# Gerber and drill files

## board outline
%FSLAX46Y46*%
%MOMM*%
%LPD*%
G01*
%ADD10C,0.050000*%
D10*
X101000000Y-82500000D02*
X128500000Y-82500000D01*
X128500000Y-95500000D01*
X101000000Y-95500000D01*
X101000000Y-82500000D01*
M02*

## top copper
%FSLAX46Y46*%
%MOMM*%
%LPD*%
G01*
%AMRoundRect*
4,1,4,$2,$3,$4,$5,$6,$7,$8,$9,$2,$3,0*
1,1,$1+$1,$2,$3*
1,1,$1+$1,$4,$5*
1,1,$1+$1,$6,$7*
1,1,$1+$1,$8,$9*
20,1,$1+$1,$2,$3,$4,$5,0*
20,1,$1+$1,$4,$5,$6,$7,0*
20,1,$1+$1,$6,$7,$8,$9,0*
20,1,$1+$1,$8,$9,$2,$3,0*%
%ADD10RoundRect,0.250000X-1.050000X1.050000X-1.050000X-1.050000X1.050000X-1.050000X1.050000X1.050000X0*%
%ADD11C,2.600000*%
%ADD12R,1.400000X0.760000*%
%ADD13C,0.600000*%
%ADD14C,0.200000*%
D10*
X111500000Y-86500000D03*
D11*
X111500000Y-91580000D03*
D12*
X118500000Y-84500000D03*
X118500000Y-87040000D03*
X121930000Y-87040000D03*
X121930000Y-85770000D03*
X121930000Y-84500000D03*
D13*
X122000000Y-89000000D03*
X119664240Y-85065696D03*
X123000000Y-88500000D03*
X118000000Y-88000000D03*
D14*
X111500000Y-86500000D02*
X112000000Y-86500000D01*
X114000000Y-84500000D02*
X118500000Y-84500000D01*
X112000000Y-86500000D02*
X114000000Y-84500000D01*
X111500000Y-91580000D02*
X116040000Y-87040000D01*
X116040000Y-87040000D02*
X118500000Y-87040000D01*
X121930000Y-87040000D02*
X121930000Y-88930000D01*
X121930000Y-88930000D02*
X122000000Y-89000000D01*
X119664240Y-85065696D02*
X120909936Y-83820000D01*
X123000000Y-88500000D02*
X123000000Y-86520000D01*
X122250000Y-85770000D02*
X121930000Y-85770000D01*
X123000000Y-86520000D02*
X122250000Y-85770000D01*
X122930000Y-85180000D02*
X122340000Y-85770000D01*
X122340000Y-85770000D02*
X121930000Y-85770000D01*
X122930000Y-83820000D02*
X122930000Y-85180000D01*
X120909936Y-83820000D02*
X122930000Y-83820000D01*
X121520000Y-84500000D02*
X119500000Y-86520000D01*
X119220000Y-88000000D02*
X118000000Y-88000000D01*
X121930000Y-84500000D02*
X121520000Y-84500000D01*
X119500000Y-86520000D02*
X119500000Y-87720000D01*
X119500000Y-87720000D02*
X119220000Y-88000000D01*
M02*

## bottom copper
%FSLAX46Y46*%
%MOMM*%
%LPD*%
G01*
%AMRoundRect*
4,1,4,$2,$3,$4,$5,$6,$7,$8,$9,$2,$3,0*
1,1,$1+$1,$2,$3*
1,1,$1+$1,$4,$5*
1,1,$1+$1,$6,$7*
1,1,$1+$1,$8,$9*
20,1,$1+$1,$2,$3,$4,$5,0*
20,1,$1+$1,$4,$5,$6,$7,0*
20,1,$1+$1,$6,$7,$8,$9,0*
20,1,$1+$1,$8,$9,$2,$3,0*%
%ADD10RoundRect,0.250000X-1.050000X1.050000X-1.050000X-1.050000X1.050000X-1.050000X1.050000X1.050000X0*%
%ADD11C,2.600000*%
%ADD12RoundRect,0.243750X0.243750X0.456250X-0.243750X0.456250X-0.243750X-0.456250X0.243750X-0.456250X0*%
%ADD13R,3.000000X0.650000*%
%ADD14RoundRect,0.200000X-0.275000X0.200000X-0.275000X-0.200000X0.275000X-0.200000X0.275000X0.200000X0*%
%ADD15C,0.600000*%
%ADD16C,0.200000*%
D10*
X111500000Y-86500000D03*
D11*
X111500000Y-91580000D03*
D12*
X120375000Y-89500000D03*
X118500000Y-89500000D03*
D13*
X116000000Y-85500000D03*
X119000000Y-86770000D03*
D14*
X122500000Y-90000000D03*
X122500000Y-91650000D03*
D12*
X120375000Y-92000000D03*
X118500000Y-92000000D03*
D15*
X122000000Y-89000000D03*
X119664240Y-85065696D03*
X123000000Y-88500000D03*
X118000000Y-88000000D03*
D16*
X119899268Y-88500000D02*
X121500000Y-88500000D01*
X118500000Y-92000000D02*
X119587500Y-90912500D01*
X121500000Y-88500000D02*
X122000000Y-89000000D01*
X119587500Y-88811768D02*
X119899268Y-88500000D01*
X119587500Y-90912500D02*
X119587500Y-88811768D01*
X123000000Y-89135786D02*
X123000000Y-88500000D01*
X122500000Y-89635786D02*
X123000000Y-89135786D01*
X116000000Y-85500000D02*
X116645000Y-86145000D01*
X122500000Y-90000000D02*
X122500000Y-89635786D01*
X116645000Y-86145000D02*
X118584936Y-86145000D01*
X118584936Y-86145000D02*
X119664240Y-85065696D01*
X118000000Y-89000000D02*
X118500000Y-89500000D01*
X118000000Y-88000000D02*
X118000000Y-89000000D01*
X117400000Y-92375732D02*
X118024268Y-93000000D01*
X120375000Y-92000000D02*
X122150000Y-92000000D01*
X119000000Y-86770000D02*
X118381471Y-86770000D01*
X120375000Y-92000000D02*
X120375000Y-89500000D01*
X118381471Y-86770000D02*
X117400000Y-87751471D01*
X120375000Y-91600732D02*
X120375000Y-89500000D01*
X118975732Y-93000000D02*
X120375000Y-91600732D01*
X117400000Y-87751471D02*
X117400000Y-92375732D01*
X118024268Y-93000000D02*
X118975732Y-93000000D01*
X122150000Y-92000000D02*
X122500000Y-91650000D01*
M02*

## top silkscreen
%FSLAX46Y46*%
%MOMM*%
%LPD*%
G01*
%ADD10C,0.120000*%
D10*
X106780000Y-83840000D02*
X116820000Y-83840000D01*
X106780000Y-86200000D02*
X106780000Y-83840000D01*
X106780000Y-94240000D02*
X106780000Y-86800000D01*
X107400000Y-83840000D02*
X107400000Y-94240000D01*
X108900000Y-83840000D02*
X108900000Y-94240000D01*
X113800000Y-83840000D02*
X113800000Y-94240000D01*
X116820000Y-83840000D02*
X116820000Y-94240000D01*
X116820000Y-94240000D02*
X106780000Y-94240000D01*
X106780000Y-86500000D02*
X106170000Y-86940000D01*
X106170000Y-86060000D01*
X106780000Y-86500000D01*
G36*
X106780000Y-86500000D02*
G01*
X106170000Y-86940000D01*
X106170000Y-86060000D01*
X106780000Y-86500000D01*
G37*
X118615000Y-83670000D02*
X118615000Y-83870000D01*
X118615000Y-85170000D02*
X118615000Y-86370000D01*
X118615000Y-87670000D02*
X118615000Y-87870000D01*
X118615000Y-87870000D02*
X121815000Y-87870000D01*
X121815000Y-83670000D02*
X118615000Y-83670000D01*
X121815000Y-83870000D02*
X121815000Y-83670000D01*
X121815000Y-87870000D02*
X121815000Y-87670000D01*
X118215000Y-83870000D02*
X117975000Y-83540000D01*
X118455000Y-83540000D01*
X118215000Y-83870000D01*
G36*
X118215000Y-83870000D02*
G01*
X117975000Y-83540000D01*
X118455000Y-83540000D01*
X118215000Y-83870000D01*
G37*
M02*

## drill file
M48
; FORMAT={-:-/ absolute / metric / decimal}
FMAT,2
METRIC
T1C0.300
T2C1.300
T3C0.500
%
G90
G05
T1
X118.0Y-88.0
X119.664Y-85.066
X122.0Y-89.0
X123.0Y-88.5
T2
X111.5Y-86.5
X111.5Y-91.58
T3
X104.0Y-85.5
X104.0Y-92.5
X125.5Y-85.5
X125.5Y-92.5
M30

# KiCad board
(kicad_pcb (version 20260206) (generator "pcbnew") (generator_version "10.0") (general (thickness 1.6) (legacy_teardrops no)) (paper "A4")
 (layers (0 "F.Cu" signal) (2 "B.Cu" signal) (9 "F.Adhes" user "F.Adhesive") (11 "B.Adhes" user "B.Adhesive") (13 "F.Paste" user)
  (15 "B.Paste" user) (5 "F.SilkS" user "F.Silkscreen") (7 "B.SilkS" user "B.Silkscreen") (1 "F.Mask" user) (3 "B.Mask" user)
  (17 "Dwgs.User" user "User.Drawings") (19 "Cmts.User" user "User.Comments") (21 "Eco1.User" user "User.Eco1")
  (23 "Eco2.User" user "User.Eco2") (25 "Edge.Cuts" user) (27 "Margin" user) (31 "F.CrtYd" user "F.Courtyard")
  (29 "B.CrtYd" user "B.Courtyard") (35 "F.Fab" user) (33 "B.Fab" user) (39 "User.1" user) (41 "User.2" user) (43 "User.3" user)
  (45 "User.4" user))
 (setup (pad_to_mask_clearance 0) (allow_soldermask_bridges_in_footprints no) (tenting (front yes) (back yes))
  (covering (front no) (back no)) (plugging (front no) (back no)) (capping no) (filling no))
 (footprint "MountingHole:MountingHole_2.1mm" (layer "F.Cu") (at 104 92.5)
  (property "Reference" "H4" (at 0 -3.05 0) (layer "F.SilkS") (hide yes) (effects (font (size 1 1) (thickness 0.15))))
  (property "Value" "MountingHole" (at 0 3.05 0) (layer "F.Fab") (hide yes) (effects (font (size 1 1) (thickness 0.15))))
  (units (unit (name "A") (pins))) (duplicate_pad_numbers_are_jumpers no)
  (pad "" np_thru_hole circle (at 0 0) (size 0.5 0.5) (drill 0.5) (layers "*.Cu" "*.Mask")))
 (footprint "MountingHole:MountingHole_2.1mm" (layer "F.Cu") (at 125.5 85.5)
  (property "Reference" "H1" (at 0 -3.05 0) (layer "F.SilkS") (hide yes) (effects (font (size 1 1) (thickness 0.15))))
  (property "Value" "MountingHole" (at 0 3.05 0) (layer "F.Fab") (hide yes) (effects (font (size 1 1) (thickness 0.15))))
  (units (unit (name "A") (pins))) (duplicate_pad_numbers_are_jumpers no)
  (pad "" np_thru_hole circle (at 0 0) (size 0.5 0.5) (drill 0.5) (layers "*.Cu" "*.Mask")))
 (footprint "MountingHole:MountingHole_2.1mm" (layer "F.Cu") (at 104 85.5)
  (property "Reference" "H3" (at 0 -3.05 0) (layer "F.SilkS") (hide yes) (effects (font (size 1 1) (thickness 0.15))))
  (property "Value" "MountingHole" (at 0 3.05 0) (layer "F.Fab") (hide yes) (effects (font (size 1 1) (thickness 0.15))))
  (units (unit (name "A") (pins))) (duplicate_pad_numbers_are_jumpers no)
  (pad "" np_thru_hole circle (at 0 0) (size 0.5 0.5) (drill 0.5) (layers "*.Cu" "*.Mask")))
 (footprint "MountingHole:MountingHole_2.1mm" (layer "F.Cu") (at 125.5 92.5)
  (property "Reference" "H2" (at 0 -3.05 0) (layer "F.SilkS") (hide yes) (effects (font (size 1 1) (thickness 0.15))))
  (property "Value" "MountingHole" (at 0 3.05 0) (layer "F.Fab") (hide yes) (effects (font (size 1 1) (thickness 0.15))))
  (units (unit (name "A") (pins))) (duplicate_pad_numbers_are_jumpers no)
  (pad "" np_thru_hole circle (at 0 0) (size 0.5 0.5) (drill 0.5) (layers "*.Cu" "*.Mask")))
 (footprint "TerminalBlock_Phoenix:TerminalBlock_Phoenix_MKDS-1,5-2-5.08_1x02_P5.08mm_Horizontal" (layer "F.Cu") (at 111.5 86.5 -90)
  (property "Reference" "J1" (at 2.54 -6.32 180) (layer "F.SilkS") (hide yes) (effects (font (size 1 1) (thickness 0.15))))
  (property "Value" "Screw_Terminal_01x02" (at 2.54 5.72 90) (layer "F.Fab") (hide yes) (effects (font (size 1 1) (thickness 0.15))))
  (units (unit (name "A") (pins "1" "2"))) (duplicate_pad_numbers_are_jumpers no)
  (fp_line (start -2.66 4.72) (end -2.66 -5.32) (stroke (width 0.12) (type solid)) (layer "F.SilkS"))
  (fp_line (start -0.3 4.72) (end -2.66 4.72) (stroke (width 0.12) (type solid)) (layer "F.SilkS"))
  (fp_line (start 7.74 4.72) (end 0.3 4.72) (stroke (width 0.12) (type solid)) (layer "F.SilkS"))
  (fp_line (start -2.66 4.1) (end 7.74 4.1) (stroke (width 0.12) (type solid)) (layer "F.SilkS"))
  (fp_line (start -2.66 2.6) (end 7.74 2.6) (stroke (width 0.12) (type solid)) (layer "F.SilkS"))
  (fp_line (start -2.66 -2.3) (end 7.74 -2.3) (stroke (width 0.12) (type solid)) (layer "F.SilkS"))
  (fp_line (start -2.66 -5.32) (end 7.74 -5.32) (stroke (width 0.12) (type solid)) (layer "F.SilkS"))
  (fp_line (start 7.74 -5.32) (end 7.74 4.72) (stroke (width 0.12) (type solid)) (layer "F.SilkS"))
  (fp_poly (pts (xy 0 4.72) (xy 0.44 5.33) (xy -0.44 5.33)) (stroke (width 0.12) (type solid)) (fill yes) (layer "F.SilkS"))
  (pad "1" thru_hole roundrect (at 0 0 270) (size 2.6 2.6) (drill 1.3) (layers "*.Cu" "*.Mask") (remove_unused_layers no)
   (roundrect_rratio 0.096154) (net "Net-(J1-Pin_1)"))
  (pad "2" thru_hole circle (at 5.08 0 270) (size 2.6 2.6) (drill 1.3) (layers "*.Cu" "*.Mask") (remove_unused_layers no)
   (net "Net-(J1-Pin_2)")))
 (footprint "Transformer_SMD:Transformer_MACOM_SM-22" (layer "F.Cu") (at 120.215 85.77)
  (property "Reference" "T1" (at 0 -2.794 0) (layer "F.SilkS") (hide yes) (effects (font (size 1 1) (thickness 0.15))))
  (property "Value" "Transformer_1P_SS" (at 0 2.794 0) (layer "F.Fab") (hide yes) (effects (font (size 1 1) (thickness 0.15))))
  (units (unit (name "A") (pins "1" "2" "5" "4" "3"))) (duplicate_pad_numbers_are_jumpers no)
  (fp_line (start -1.6 -2.1) (end -1.6 -1.9) (stroke (width 0.12) (type solid)) (layer "F.SilkS"))
  (fp_line (start -1.6 -0.6) (end -1.6 0.6) (stroke (width 0.12) (type solid)) (layer "F.SilkS"))
  (fp_line (start -1.6 1.9) (end -1.6 2.1) (stroke (width 0.12) (type solid)) (layer "F.SilkS"))
  (fp_line (start -1.6 2.1) (end 1.6 2.1) (stroke (width 0.12) (type solid)) (layer "F.SilkS"))
  (fp_line (start 1.6 -2.1) (end -1.6 -2.1) (stroke (width 0.12) (type solid)) (layer "F.SilkS"))
  (fp_line (start 1.6 -1.9) (end 1.6 -2.1) (stroke (width 0.12) (type solid)) (layer "F.SilkS"))
  (fp_line (start 1.6 2.1) (end 1.6 1.9) (stroke (width 0.12) (type solid)) (layer "F.SilkS"))
  (fp_poly
   (pts (xy -2 -1.9) (xy -2.24 -2.23) (xy -1.76 -2.23) (xy -2 -1.9)) (stroke (width 0.12) (type solid)) (fill yes) (layer "F.SilkS"))
  (pad "1" smd rect (at -1.715 -1.27) (size 1.4 0.76) (layers "F.Cu" "F.Mask" "F.Paste") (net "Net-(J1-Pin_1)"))
  (pad "2" smd rect (at -1.715 1.27) (size 1.4 0.76) (layers "F.Cu" "F.Mask" "F.Paste") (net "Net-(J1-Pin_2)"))
  (pad "3" smd rect (at 1.715 1.27) (size 1.4 0.76) (layers "F.Cu" "F.Mask" "F.Paste") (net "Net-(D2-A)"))
  (pad "4" smd rect (at 1.715 0) (size 1.4 0.76) (layers "F.Cu" "F.Mask" "F.Paste") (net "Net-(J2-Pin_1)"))
  (pad "5" smd rect (at 1.715 -1.27) (size 1.4 0.76) (layers "F.Cu" "F.Mask" "F.Paste") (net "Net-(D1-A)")))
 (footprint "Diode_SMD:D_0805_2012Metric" (layer "B.Cu") (at 119.4375 89.5 180)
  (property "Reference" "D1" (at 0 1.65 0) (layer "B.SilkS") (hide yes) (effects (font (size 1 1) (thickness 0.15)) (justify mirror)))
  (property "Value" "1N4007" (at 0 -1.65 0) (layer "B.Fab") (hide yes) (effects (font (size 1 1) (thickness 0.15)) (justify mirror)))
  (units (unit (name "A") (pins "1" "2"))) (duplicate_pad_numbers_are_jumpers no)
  (pad "1" smd roundrect (at -0.9375 0 180) (size 0.975 1.4) (layers "B.Cu" "B.Mask" "B.Paste") (roundrect_rratio 0.25) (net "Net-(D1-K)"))
  (pad "2" smd roundrect (at 0.9375 0 180) (size 0.975 1.4) (layers "B.Cu" "B.Mask" "B.Paste") (roundrect_rratio 0.25) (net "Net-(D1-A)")))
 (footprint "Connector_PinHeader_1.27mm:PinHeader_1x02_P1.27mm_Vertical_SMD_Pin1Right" (layer "B.Cu") (at 117.5 86.135 180)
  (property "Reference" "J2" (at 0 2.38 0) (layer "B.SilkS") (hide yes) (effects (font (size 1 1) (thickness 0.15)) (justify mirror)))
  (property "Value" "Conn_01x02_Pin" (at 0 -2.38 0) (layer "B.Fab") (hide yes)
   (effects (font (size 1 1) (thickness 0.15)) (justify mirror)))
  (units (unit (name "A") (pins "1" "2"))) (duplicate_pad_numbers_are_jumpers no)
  (pad "1" smd rect (at 1.5 0.635 180) (size 3 0.65) (layers "B.Cu" "B.Mask" "B.Paste") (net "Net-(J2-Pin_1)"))
  (pad "2" smd rect (at -1.5 -0.635 180) (size 3 0.65) (layers "B.Cu" "B.Mask" "B.Paste") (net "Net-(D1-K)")))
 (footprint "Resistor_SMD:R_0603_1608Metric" (layer "B.Cu") (at 122.5 90.825 -90)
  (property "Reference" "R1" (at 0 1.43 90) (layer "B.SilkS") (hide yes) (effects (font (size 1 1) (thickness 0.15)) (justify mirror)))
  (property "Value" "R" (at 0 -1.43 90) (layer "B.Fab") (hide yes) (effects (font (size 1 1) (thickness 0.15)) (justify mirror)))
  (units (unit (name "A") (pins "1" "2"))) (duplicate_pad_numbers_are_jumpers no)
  (pad "1" smd roundrect (at -0.825 0 270) (size 0.8 0.95) (layers "B.Cu" "B.Mask" "B.Paste") (roundrect_rratio 0.25) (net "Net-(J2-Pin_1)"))
  (pad "2" smd roundrect (at 0.825 0 270) (size 0.8 0.95) (layers "B.Cu" "B.Mask" "B.Paste") (roundrect_rratio 0.25) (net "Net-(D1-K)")))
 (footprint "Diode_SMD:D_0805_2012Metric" (layer "B.Cu") (at 119.4375 92 180)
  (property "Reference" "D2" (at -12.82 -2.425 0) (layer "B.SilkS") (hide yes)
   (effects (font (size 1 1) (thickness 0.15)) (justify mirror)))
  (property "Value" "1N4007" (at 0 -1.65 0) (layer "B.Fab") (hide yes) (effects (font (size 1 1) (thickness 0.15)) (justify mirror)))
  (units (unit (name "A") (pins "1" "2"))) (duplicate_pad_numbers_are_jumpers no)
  (pad "1" smd roundrect (at -0.9375 0 180) (size 0.975 1.4) (layers "B.Cu" "B.Mask" "B.Paste") (roundrect_rratio 0.25) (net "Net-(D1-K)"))
  (pad "2" smd roundrect (at 0.9375 0 180) (size 0.975 1.4) (layers "B.Cu" "B.Mask" "B.Paste") (roundrect_rratio 0.25) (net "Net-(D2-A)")))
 (gr_rect (start 101 82.5) (end 128.5 95.5) (stroke (width 0.05) (type default)) (fill no) (layer "Edge.Cuts"))
 (segment (start 111.5 86.5) (end 112 86.5) (width 0.2) (layer "F.Cu") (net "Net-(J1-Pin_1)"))
 (segment (start 114 84.5) (end 118.5 84.5) (width 0.2) (layer "F.Cu") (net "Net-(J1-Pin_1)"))
 (segment (start 112 86.5) (end 114 84.5) (width 0.2) (layer "F.Cu") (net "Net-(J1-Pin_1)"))
 (segment (start 111.5 91.58) (end 116.04 87.04) (width 0.2) (layer "F.Cu") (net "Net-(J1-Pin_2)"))
 (segment (start 116.04 87.04) (end 118.5 87.04) (width 0.2) (layer "F.Cu") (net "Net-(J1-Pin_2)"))
 (segment (start 121.93 87.04) (end 121.93 88.93) (width 0.2) (layer "F.Cu") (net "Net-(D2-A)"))
 (segment (start 121.93 88.93) (end 122 89) (width 0.2) (layer "F.Cu") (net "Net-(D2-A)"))
 (via (at 122 89) (size 0.6) (drill 0.3) (layers "F.Cu" "B.Cu") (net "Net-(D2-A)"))
 (segment (start 119.899268 88.5) (end 121.5 88.5) (width 0.2) (layer "B.Cu") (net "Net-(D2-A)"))
 (segment (start 118.5 92) (end 119.5875 90.9125) (width 0.2) (layer "B.Cu") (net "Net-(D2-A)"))
 (segment (start 121.5 88.5) (end 122 89) (width 0.2) (layer "B.Cu") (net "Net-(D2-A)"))
 (segment (start 119.5875 88.811768) (end 119.899268 88.5) (width 0.2) (layer "B.Cu") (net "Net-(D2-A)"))
 (segment (start 119.5875 90.9125) (end 119.5875 88.811768) (width 0.2) (layer "B.Cu") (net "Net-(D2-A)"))
 (segment (start 119.66424 85.065696) (end 120.909936 83.82) (width 0.2) (layer "F.Cu") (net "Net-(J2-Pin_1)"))
 (segment (start 123 88.5) (end 123 86.52) (width 0.2) (layer "F.Cu") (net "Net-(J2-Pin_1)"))
 (segment (start 122.25 85.77) (end 121.93 85.77) (width 0.2) (layer "F.Cu") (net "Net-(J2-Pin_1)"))
 (segment (start 123 86.52) (end 122.25 85.77) (width 0.2) (layer "F.Cu") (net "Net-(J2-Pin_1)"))
 (segment (start 122.93 85.18) (end 122.34 85.77) (width 0.2) (layer "F.Cu") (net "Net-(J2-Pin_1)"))
 (segment (start 122.34 85.77) (end 121.93 85.77) (width 0.2) (layer "F.Cu") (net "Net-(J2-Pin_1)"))
 (segment (start 122.93 83.82) (end 122.93 85.18) (width 0.2) (layer "F.Cu") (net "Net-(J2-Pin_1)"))
 (segment (start 120.909936 83.82) (end 122.93 83.82) (width 0.2) (layer "F.Cu") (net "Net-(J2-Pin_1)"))
 (via (at 119.66424 85.065696) (size 0.6) (drill 0.3) (layers "F.Cu" "B.Cu") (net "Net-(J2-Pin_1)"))
 (via (at 123 88.5) (size 0.6) (drill 0.3) (layers "F.Cu" "B.Cu") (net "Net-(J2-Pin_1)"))
 (segment (start 123 89.135786) (end 123 88.5) (width 0.2) (layer "B.Cu") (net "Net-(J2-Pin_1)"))
 (segment (start 122.5 89.635786) (end 123 89.135786) (width 0.2) (layer "B.Cu") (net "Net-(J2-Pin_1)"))
 (segment (start 116 85.5) (end 116.645 86.145) (width 0.2) (layer "B.Cu") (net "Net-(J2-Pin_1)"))
 (segment (start 122.5 90) (end 122.5 89.635786) (width 0.2) (layer "B.Cu") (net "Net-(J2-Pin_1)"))
 (segment (start 116.645 86.145) (end 118.584936 86.145) (width 0.2) (layer "B.Cu") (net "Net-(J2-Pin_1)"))
 (segment (start 118.584936 86.145) (end 119.66424 85.065696) (width 0.2) (layer "B.Cu") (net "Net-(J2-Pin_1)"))
 (segment (start 121.52 84.5) (end 119.5 86.52) (width 0.2) (layer "F.Cu") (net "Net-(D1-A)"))
 (segment (start 119.22 88) (end 118 88) (width 0.2) (layer "F.Cu") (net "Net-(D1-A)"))
 (segment (start 121.93 84.5) (end 121.52 84.5) (width 0.2) (layer "F.Cu") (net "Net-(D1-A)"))
 (segment (start 119.5 86.52) (end 119.5 87.72) (width 0.2) (layer "F.Cu") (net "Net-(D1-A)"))
 (segment (start 119.5 87.72) (end 119.22 88) (width 0.2) (layer "F.Cu") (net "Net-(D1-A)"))
 (via (at 118 88) (size 0.6) (drill 0.3) (layers "F.Cu" "B.Cu") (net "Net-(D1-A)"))
 (segment (start 118 89) (end 118.5 89.5) (width 0.2) (layer "B.Cu") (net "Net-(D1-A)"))
 (segment (start 118 88) (end 118 89) (width 0.2) (layer "B.Cu") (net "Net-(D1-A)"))
 (segment (start 117.4 92.375732) (end 118.024268 93) (width 0.2) (layer "B.Cu") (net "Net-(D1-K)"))
 (segment (start 120.375 92) (end 122.15 92) (width 0.2) (layer "B.Cu") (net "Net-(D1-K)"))
 (segment (start 119 86.77) (end 118.381471 86.77) (width 0.2) (layer "B.Cu") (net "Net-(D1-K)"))
 (segment (start 120.375 92) (end 120.375 89.5) (width 0.2) (layer "B.Cu") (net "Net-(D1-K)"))
 (segment (start 118.381471 86.77) (end 117.4 87.751471) (width 0.2) (layer "B.Cu") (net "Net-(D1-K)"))
 (segment (start 120.375 91.600732) (end 120.375 89.5) (width 0.2) (layer "B.Cu") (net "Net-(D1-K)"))
 (segment (start 118.975732 93) (end 120.375 91.600732) (width 0.2) (layer "B.Cu") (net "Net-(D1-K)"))
 (segment (start 117.4 87.751471) (end 117.4 92.375732) (width 0.2) (layer "B.Cu") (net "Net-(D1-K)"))
 (segment (start 118.024268 93) (end 118.975732 93) (width 0.2) (layer "B.Cu") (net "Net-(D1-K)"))
 (segment (start 122.15 92) (end 122.5 91.65) (width 0.2) (layer "B.Cu") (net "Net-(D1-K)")))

